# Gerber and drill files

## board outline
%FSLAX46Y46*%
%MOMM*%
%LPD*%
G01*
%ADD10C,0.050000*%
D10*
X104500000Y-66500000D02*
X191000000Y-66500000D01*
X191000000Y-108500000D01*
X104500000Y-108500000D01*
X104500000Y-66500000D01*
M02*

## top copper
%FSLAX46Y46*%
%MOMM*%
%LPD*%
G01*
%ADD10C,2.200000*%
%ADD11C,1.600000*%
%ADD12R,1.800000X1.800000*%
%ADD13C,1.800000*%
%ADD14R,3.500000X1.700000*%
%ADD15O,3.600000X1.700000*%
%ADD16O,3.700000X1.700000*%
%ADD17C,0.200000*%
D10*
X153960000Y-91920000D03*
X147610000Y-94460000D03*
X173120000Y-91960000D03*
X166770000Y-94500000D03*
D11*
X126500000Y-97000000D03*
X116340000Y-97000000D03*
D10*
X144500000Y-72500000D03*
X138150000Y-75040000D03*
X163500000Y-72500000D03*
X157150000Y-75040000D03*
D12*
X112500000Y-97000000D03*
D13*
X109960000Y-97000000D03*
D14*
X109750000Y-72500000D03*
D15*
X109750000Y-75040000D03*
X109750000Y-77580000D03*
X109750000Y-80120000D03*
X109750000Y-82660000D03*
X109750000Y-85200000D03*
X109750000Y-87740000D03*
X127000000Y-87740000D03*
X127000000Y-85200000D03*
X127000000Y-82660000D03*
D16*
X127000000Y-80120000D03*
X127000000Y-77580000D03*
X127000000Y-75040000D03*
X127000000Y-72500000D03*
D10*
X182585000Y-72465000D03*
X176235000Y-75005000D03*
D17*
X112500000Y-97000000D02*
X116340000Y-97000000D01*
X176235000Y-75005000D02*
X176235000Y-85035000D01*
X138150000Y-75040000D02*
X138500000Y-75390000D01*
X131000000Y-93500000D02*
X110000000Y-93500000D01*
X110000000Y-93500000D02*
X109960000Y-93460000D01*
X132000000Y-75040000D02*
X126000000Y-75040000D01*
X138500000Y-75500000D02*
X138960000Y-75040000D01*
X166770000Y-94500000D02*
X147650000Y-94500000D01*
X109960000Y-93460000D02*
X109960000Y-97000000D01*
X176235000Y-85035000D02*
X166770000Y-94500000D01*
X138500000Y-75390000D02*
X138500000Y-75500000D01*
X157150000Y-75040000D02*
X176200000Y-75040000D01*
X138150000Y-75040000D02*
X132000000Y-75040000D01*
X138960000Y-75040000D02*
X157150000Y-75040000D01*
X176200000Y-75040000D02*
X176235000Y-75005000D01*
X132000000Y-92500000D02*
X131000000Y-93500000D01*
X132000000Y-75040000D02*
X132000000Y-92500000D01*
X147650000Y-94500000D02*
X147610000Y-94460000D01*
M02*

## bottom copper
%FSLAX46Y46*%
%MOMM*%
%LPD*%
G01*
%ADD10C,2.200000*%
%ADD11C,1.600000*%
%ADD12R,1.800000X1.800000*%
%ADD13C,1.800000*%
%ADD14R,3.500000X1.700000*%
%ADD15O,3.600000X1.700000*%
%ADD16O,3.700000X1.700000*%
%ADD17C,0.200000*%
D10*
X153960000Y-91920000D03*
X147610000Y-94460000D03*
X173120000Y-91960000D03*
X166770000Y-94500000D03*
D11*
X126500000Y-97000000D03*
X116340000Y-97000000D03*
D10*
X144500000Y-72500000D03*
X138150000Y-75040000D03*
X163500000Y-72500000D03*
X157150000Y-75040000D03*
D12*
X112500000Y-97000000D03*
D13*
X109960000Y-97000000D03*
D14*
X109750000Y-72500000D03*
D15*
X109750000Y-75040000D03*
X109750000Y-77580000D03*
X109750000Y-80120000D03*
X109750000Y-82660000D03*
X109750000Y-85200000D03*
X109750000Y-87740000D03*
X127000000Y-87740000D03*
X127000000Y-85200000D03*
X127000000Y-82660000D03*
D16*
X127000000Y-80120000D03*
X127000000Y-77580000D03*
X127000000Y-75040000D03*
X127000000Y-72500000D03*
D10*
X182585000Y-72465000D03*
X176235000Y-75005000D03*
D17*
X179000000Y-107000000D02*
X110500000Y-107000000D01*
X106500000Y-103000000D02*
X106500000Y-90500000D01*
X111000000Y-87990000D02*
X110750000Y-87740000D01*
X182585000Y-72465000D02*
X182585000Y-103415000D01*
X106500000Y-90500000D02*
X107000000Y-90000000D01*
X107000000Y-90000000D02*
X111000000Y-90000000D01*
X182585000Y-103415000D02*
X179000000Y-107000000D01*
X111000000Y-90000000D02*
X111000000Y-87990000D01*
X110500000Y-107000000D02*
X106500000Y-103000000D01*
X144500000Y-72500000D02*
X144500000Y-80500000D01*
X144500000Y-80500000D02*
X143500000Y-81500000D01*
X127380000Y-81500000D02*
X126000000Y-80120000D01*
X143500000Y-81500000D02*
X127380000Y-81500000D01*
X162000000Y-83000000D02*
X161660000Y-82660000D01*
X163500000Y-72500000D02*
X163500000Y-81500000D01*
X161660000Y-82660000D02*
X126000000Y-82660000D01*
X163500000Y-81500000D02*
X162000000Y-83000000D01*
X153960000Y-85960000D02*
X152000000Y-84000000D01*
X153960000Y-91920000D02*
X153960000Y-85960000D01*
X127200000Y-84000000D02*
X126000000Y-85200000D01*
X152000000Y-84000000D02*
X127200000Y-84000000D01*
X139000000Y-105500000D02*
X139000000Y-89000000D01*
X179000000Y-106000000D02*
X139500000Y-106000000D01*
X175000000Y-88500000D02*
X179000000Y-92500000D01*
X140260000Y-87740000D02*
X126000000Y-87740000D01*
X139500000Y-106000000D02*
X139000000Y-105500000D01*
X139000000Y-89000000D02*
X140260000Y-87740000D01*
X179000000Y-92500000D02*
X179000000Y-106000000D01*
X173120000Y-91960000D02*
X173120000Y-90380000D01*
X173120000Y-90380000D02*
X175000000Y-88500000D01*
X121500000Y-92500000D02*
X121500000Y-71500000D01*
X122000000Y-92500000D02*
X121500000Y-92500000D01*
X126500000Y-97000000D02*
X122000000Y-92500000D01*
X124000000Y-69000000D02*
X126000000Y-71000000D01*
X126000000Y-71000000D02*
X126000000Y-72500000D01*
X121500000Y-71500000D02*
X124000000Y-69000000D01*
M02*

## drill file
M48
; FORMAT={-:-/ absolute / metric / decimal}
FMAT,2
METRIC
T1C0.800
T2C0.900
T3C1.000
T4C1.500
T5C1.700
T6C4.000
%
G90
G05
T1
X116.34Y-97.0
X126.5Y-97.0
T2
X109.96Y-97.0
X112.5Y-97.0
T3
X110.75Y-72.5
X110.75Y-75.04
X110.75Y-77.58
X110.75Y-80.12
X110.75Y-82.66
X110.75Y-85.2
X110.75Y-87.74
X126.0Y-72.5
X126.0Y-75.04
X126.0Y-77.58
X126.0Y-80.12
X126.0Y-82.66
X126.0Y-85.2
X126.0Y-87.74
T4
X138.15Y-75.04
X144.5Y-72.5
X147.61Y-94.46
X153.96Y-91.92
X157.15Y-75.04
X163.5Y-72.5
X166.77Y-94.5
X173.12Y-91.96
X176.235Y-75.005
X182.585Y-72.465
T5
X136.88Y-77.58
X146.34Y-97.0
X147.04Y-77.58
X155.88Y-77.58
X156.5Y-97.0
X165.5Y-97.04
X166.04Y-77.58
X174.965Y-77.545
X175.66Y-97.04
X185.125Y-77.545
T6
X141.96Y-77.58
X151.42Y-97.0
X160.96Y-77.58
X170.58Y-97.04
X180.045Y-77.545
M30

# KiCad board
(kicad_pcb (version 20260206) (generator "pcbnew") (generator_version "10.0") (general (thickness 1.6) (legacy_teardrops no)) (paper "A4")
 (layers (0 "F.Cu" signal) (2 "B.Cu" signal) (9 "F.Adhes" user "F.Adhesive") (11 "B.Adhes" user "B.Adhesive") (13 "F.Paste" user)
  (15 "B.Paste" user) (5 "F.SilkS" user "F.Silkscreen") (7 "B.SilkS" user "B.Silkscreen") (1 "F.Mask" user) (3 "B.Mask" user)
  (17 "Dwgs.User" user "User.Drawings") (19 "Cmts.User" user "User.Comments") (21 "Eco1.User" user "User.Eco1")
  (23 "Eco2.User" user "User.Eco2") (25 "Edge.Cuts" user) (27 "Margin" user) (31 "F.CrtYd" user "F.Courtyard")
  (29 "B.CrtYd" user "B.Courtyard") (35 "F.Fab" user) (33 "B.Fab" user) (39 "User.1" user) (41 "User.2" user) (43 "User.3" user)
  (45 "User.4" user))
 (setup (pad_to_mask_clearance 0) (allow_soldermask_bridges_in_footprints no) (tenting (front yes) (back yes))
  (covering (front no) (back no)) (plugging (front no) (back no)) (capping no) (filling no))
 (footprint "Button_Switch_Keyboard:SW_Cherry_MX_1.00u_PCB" (layer "F.Cu") (at 153.96 91.92)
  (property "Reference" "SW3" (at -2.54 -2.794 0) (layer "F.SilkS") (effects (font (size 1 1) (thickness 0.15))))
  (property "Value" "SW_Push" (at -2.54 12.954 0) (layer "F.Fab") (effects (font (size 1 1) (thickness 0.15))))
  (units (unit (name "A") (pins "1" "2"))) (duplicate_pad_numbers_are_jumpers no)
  (pad "" np_thru_hole circle (at -7.62 5.08) (size 1.7 1.7) (drill 1.7) (layers "*.Cu" "*.Mask"))
  (pad "" np_thru_hole circle (at -2.54 5.08) (size 4 4) (drill 4) (layers "*.Cu" "*.Mask"))
  (pad "" np_thru_hole circle (at 2.54 5.08) (size 1.7 1.7) (drill 1.7) (layers "*.Cu" "*.Mask"))
  (pad "1" thru_hole circle (at 0 0) (size 2.2 2.2) (drill 1.5) (layers "*.Cu" "*.Mask") (remove_unused_layers no)
   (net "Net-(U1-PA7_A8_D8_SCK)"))
  (pad "2" thru_hole circle (at -6.35 2.54) (size 2.2 2.2) (drill 1.5) (layers "*.Cu" "*.Mask") (remove_unused_layers no) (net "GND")))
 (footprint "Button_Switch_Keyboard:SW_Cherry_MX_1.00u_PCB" (layer "F.Cu") (at 173.12 91.96)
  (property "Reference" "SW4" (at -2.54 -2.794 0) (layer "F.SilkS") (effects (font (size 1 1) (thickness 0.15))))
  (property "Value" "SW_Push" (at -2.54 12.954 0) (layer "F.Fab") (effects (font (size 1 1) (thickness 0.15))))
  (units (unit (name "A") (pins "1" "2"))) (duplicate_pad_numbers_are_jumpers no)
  (pad "" np_thru_hole circle (at -7.62 5.08) (size 1.7 1.7) (drill 1.7) (layers "*.Cu" "*.Mask"))
  (pad "" np_thru_hole circle (at -2.54 5.08) (size 4 4) (drill 4) (layers "*.Cu" "*.Mask"))
  (pad "" np_thru_hole circle (at 2.54 5.08) (size 1.7 1.7) (drill 1.7) (layers "*.Cu" "*.Mask"))
  (pad "1" thru_hole circle (at 0 0) (size 2.2 2.2) (drill 1.5) (layers "*.Cu" "*.Mask") (remove_unused_layers no)
   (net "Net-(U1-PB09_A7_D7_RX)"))
  (pad "2" thru_hole circle (at -6.35 2.54) (size 2.2 2.2) (drill 1.5) (layers "*.Cu" "*.Mask") (remove_unused_layers no) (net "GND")))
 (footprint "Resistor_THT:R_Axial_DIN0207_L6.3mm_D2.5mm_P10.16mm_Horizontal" (layer "F.Cu") (at 126.5 97 180)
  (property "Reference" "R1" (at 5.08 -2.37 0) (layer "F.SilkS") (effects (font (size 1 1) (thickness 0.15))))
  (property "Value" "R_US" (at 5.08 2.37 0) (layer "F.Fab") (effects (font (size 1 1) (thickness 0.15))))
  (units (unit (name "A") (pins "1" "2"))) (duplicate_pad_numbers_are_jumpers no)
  (pad "1" thru_hole circle (at 0 0 180) (size 1.6 1.6) (drill 0.8) (layers "*.Cu" "*.Mask") (remove_unused_layers no) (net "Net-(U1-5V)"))
  (pad "2" thru_hole circle (at 10.16 0 180) (size 1.6 1.6) (drill 0.8) (layers "*.Cu" "*.Mask") (remove_unused_layers no)
   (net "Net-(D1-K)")))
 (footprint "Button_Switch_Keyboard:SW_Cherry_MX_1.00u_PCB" (layer "F.Cu") (at 144.5 72.5)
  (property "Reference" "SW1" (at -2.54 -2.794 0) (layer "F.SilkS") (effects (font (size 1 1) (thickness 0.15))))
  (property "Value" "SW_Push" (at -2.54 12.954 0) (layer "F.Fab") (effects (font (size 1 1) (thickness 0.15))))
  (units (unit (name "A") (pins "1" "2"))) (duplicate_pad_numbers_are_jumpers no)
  (pad "" np_thru_hole circle (at -7.62 5.08) (size 1.7 1.7) (drill 1.7) (layers "*.Cu" "*.Mask"))
  (pad "" np_thru_hole circle (at -2.54 5.08) (size 4 4) (drill 4) (layers "*.Cu" "*.Mask"))
  (pad "" np_thru_hole circle (at 2.54 5.08) (size 1.7 1.7) (drill 1.7) (layers "*.Cu" "*.Mask"))
  (pad "1" thru_hole circle (at 0 0) (size 2.2 2.2) (drill 1.5) (layers "*.Cu" "*.Mask") (remove_unused_layers no)
   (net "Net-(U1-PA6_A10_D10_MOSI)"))
  (pad "2" thru_hole circle (at -6.35 2.54) (size 2.2 2.2) (drill 1.5) (layers "*.Cu" "*.Mask") (remove_unused_layers no) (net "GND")))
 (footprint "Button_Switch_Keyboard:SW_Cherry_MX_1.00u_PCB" (layer "F.Cu") (at 163.5 72.5)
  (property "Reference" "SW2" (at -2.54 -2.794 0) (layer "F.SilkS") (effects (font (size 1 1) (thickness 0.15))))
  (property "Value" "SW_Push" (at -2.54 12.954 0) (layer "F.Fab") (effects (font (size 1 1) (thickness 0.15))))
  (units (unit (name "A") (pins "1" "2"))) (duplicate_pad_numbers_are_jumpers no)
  (pad "" np_thru_hole circle (at -7.62 5.08) (size 1.7 1.7) (drill 1.7) (layers "*.Cu" "*.Mask"))
  (pad "" np_thru_hole circle (at -2.54 5.08) (size 4 4) (drill 4) (layers "*.Cu" "*.Mask"))
  (pad "" np_thru_hole circle (at 2.54 5.08) (size 1.7 1.7) (drill 1.7) (layers "*.Cu" "*.Mask"))
  (pad "1" thru_hole circle (at 0 0) (size 2.2 2.2) (drill 1.5) (layers "*.Cu" "*.Mask") (remove_unused_layers no)
   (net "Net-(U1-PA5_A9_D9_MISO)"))
  (pad "2" thru_hole circle (at -6.35 2.54) (size 2.2 2.2) (drill 1.5) (layers "*.Cu" "*.Mask") (remove_unused_layers no) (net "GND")))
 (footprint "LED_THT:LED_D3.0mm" (layer "F.Cu") (at 112.5 97 180)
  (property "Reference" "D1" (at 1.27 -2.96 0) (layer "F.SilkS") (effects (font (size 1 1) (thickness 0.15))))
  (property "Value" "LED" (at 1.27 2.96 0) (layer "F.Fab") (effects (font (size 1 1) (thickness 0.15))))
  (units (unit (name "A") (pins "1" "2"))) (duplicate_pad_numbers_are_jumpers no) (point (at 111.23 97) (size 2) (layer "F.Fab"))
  (pad "1" thru_hole rect (at 0 0 180) (size 1.8 1.8) (drill 0.9) (layers "*.Cu" "*.Mask") (remove_unused_layers no) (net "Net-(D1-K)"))
  (pad "2" thru_hole circle (at 2.54 0 180) (size 1.8 1.8) (drill 0.9) (layers "*.Cu" "*.Mask") (remove_unused_layers no) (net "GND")))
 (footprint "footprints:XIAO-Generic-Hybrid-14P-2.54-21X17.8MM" (layer "F.Cu") (at 118.375 80.12)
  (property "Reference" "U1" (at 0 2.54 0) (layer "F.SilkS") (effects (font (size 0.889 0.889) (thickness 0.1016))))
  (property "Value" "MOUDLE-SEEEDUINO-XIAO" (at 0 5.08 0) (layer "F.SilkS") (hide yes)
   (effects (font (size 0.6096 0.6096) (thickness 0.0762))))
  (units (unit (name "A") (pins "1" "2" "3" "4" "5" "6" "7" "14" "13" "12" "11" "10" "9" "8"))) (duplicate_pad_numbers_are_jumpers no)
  (pad "1" thru_hole rect (at -7.625 -7.62) (size 3.5 1.7) (drill 1 (offset -1 0)) (layers "*.Cu" "*.Mask") (remove_unused_layers no)
   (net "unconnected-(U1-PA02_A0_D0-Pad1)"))
  (pad "2" thru_hole oval (at -7.625 -5.08) (size 3.6 1.7) (drill 1 (offset -1 0)) (layers "*.Cu" "*.Mask") (remove_unused_layers no)
   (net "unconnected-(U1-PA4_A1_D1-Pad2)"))
  (pad "3" thru_hole oval (at -7.625 -2.54) (size 3.6 1.7) (drill 1 (offset -1 0)) (layers "*.Cu" "*.Mask") (remove_unused_layers no)
   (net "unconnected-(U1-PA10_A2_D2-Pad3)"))
  (pad "4" thru_hole oval (at -7.625 0) (size 3.6 1.7) (drill 1 (offset -1 0)) (layers "*.Cu" "*.Mask") (remove_unused_layers no)
   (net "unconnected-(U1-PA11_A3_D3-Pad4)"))
  (pad "5" thru_hole oval (at -7.625 2.54) (size 3.6 1.7) (drill 1 (offset -1 0)) (layers "*.Cu" "*.Mask") (remove_unused_layers no)
   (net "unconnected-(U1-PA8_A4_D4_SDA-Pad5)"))
  (pad "6" thru_hole oval (at -7.625 5.08 180) (size 3.6 1.7) (drill 1 (offset 1 0)) (layers "*.Cu" "*.Mask") (remove_unused_layers no)
   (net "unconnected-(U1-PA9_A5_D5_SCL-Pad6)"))
  (pad "7" thru_hole oval (at -7.625 7.62) (size 3.6 1.7) (drill 1 (offset -1 0)) (layers "*.Cu" "*.Mask") (remove_unused_layers no)
   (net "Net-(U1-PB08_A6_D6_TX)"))
  (pad "8" thru_hole oval (at 7.625 7.62) (size 3.6 1.7) (drill 1 (offset 1 0)) (layers "*.Cu" "*.Mask") (remove_unused_layers no)
   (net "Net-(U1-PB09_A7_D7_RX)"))
  (pad "9" thru_hole oval (at 7.625 5.08) (size 3.6 1.7) (drill 1 (offset 1 0)) (layers "*.Cu" "*.Mask") (remove_unused_layers no)
   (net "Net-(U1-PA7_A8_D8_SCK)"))
  (pad "10" thru_hole oval (at 7.625 2.54) (size 3.6 1.7) (drill 1 (offset 1 0)) (layers "*.Cu" "*.Mask") (remove_unused_layers no)
   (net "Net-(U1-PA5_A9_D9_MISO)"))
  (pad "11" thru_hole oval (at 7.625 0) (size 3.7 1.7) (drill 1 (offset 1 0)) (layers "*.Cu" "*.Mask") (remove_unused_layers no)
   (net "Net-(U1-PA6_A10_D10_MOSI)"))
  (pad "12" thru_hole oval (at 7.625 -2.54) (size 3.7 1.7) (drill 1 (offset 1 0)) (layers "*.Cu" "*.Mask") (remove_unused_layers no)
   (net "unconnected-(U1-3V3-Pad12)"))
  (pad "13" thru_hole oval (at 7.625 -5.08) (size 3.7 1.7) (drill 1 (offset 1 0)) (layers "*.Cu" "*.Mask") (remove_unused_layers no)
   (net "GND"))
  (pad "14" thru_hole oval (at 7.625 -7.62) (size 3.7 1.7) (drill 1 (offset 1 0)) (layers "*.Cu" "*.Mask") (remove_unused_layers no)
   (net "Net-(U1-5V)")))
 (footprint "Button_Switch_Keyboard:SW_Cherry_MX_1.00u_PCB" (layer "F.Cu") (at 182.585 72.465)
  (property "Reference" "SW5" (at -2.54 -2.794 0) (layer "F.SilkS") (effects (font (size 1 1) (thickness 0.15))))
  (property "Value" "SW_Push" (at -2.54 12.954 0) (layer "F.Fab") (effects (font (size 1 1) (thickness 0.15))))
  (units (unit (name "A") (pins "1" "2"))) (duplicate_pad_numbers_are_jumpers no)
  (pad "" np_thru_hole circle (at -7.62 5.08) (size 1.7 1.7) (drill 1.7) (layers "*.Cu" "*.Mask"))
  (pad "" np_thru_hole circle (at -2.54 5.08) (size 4 4) (drill 4) (layers "*.Cu" "*.Mask"))
  (pad "" np_thru_hole circle (at 2.54 5.08) (size 1.7 1.7) (drill 1.7) (layers "*.Cu" "*.Mask"))
  (pad "1" thru_hole circle (at 0 0) (size 2.2 2.2) (drill 1.5) (layers "*.Cu" "*.Mask") (remove_unused_layers no)
   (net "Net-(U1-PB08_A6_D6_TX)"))
  (pad "2" thru_hole circle (at -6.35 2.54) (size 2.2 2.2) (drill 1.5) (layers "*.Cu" "*.Mask") (remove_unused_layers no) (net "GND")))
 (gr_rect (start 104.5 66.5) (end 191 108.5) (stroke (width 0.05) (type default)) (fill no) (layer "Edge.Cuts"))
 (segment (start 112.5 97) (end 116.34 97) (width 0.2) (layer "F.Cu") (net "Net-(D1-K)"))
 (segment (start 176.235 75.005) (end 176.235 85.035) (width 0.2) (layer "F.Cu") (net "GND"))
 (segment (start 138.15 75.04) (end 138.5 75.39) (width 0.2) (layer "F.Cu") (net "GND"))
 (segment (start 131 93.5) (end 110 93.5) (width 0.2) (layer "F.Cu") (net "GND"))
 (segment (start 110 93.5) (end 109.96 93.46) (width 0.2) (layer "F.Cu") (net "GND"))
 (segment (start 132 75.04) (end 126 75.04) (width 0.2) (layer "F.Cu") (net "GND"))
 (segment (start 138.5 75.5) (end 138.96 75.04) (width 0.2) (layer "F.Cu") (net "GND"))
 (segment (start 166.77 94.5) (end 147.65 94.5) (width 0.2) (layer "F.Cu") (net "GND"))
 (segment (start 109.96 93.46) (end 109.96 97) (width 0.2) (layer "F.Cu") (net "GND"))
 (segment (start 176.235 85.035) (end 166.77 94.5) (width 0.2) (layer "F.Cu") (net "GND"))
 (segment (start 138.5 75.39) (end 138.5 75.5) (width 0.2) (layer "F.Cu") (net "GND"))
 (segment (start 157.15 75.04) (end 176.2 75.04) (width 0.2) (layer "F.Cu") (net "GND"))
 (segment (start 138.15 75.04) (end 132 75.04) (width 0.2) (layer "F.Cu") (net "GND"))
 (segment (start 138.96 75.04) (end 157.15 75.04) (width 0.2) (layer "F.Cu") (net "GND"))
 (segment (start 176.2 75.04) (end 176.235 75.005) (width 0.2) (layer "F.Cu") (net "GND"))
 (segment (start 132 92.5) (end 131 93.5) (width 0.2) (layer "F.Cu") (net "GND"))
 (segment (start 132 75.04) (end 132 92.5) (width 0.2) (layer "F.Cu") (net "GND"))
 (segment (start 147.65 94.5) (end 147.61 94.46) (width 0.2) (layer "F.Cu") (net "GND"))
 (segment (start 179 107) (end 110.5 107) (width 0.2) (layer "B.Cu") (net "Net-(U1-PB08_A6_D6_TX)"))
 (segment (start 106.5 103) (end 106.5 90.5) (width 0.2) (layer "B.Cu") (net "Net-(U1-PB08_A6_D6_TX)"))
 (segment (start 111 87.99) (end 110.75 87.74) (width 0.2) (layer "B.Cu") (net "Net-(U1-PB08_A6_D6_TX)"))
 (segment (start 182.585 72.465) (end 182.585 103.415) (width 0.2) (layer "B.Cu") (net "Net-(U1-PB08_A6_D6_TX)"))
 (segment (start 106.5 90.5) (end 107 90) (width 0.2) (layer "B.Cu") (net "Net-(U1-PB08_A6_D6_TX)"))
 (segment (start 107 90) (end 111 90) (width 0.2) (layer "B.Cu") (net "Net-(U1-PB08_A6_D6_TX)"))
 (segment (start 182.585 103.415) (end 179 107) (width 0.2) (layer "B.Cu") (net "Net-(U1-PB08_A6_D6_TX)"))
 (segment (start 111 90) (end 111 87.99) (width 0.2) (layer "B.Cu") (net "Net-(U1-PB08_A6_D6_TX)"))
 (segment (start 110.5 107) (end 106.5 103) (width 0.2) (layer "B.Cu") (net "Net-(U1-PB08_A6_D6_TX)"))
 (segment (start 144.5 72.5) (end 144.5 80.5) (width 0.2) (layer "B.Cu") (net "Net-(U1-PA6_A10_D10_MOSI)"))
 (segment (start 144.5 80.5) (end 143.5 81.5) (width 0.2) (layer "B.Cu") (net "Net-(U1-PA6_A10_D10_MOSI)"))
 (segment (start 127.38 81.5) (end 126 80.12) (width 0.2) (layer "B.Cu") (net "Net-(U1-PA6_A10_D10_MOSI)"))
 (segment (start 143.5 81.5) (end 127.38 81.5) (width 0.2) (layer "B.Cu") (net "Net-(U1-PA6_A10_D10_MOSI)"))
 (segment (start 162 83) (end 161.66 82.66) (width 0.2) (layer "B.Cu") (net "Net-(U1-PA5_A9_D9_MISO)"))
 (segment (start 163.5 72.5) (end 163.5 81.5) (width 0.2) (layer "B.Cu") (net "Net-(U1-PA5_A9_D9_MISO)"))
 (segment (start 161.66 82.66) (end 126 82.66) (width 0.2) (layer "B.Cu") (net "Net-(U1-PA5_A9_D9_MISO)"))
 (segment (start 163.5 81.5) (end 162 83) (width 0.2) (layer "B.Cu") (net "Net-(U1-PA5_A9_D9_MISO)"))
 (segment (start 153.96 85.96) (end 152 84) (width 0.2) (layer "B.Cu") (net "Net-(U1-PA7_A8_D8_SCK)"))
 (segment (start 153.96 91.92) (end 153.96 85.96) (width 0.2) (layer "B.Cu") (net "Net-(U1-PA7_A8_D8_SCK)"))
 (segment (start 127.2 84) (end 126 85.2) (width 0.2) (layer "B.Cu") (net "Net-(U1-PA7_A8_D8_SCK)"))
 (segment (start 152 84) (end 127.2 84) (width 0.2) (layer "B.Cu") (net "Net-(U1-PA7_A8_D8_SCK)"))
 (segment (start 139 105.5) (end 139 89) (width 0.2) (layer "B.Cu") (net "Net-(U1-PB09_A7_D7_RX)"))
 (segment (start 179 106) (end 139.5 106) (width 0.2) (layer "B.Cu") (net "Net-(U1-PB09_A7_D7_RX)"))
 (segment (start 175 88.5) (end 179 92.5) (width 0.2) (layer "B.Cu") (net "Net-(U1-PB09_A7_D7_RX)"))
 (segment (start 140.26 87.74) (end 126 87.74) (width 0.2) (layer "B.Cu") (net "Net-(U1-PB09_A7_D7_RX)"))
 (segment (start 139.5 106) (end 139 105.5) (width 0.2) (layer "B.Cu") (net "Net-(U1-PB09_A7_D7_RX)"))
 (segment (start 139 89) (end 140.26 87.74) (width 0.2) (layer "B.Cu") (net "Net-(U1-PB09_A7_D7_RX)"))
 (segment (start 179 92.5) (end 179 106) (width 0.2) (layer "B.Cu") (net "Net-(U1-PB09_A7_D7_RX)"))
 (segment (start 173.12 91.96) (end 173.12 90.38) (width 0.2) (layer "B.Cu") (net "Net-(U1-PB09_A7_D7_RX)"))
 (segment (start 173.12 90.38) (end 175 88.5) (width 0.2) (layer "B.Cu") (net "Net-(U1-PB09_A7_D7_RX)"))
 (segment (start 121.5 92.5) (end 121.5 71.5) (width 0.2) (layer "B.Cu") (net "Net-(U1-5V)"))
 (segment (start 122 92.5) (end 121.5 92.5) (width 0.2) (layer "B.Cu") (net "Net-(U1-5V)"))
 (segment (start 126.5 97) (end 122 92.5) (width 0.2) (layer "B.Cu") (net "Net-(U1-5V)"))
 (segment (start 124 69) (end 126 71) (width 0.2) (layer "B.Cu") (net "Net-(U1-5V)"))
 (segment (start 126 71) (end 126 72.5) (width 0.2) (layer "B.Cu") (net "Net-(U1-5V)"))
 (segment (start 121.5 71.5) (end 124 69) (width 0.2) (layer "B.Cu") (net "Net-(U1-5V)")))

